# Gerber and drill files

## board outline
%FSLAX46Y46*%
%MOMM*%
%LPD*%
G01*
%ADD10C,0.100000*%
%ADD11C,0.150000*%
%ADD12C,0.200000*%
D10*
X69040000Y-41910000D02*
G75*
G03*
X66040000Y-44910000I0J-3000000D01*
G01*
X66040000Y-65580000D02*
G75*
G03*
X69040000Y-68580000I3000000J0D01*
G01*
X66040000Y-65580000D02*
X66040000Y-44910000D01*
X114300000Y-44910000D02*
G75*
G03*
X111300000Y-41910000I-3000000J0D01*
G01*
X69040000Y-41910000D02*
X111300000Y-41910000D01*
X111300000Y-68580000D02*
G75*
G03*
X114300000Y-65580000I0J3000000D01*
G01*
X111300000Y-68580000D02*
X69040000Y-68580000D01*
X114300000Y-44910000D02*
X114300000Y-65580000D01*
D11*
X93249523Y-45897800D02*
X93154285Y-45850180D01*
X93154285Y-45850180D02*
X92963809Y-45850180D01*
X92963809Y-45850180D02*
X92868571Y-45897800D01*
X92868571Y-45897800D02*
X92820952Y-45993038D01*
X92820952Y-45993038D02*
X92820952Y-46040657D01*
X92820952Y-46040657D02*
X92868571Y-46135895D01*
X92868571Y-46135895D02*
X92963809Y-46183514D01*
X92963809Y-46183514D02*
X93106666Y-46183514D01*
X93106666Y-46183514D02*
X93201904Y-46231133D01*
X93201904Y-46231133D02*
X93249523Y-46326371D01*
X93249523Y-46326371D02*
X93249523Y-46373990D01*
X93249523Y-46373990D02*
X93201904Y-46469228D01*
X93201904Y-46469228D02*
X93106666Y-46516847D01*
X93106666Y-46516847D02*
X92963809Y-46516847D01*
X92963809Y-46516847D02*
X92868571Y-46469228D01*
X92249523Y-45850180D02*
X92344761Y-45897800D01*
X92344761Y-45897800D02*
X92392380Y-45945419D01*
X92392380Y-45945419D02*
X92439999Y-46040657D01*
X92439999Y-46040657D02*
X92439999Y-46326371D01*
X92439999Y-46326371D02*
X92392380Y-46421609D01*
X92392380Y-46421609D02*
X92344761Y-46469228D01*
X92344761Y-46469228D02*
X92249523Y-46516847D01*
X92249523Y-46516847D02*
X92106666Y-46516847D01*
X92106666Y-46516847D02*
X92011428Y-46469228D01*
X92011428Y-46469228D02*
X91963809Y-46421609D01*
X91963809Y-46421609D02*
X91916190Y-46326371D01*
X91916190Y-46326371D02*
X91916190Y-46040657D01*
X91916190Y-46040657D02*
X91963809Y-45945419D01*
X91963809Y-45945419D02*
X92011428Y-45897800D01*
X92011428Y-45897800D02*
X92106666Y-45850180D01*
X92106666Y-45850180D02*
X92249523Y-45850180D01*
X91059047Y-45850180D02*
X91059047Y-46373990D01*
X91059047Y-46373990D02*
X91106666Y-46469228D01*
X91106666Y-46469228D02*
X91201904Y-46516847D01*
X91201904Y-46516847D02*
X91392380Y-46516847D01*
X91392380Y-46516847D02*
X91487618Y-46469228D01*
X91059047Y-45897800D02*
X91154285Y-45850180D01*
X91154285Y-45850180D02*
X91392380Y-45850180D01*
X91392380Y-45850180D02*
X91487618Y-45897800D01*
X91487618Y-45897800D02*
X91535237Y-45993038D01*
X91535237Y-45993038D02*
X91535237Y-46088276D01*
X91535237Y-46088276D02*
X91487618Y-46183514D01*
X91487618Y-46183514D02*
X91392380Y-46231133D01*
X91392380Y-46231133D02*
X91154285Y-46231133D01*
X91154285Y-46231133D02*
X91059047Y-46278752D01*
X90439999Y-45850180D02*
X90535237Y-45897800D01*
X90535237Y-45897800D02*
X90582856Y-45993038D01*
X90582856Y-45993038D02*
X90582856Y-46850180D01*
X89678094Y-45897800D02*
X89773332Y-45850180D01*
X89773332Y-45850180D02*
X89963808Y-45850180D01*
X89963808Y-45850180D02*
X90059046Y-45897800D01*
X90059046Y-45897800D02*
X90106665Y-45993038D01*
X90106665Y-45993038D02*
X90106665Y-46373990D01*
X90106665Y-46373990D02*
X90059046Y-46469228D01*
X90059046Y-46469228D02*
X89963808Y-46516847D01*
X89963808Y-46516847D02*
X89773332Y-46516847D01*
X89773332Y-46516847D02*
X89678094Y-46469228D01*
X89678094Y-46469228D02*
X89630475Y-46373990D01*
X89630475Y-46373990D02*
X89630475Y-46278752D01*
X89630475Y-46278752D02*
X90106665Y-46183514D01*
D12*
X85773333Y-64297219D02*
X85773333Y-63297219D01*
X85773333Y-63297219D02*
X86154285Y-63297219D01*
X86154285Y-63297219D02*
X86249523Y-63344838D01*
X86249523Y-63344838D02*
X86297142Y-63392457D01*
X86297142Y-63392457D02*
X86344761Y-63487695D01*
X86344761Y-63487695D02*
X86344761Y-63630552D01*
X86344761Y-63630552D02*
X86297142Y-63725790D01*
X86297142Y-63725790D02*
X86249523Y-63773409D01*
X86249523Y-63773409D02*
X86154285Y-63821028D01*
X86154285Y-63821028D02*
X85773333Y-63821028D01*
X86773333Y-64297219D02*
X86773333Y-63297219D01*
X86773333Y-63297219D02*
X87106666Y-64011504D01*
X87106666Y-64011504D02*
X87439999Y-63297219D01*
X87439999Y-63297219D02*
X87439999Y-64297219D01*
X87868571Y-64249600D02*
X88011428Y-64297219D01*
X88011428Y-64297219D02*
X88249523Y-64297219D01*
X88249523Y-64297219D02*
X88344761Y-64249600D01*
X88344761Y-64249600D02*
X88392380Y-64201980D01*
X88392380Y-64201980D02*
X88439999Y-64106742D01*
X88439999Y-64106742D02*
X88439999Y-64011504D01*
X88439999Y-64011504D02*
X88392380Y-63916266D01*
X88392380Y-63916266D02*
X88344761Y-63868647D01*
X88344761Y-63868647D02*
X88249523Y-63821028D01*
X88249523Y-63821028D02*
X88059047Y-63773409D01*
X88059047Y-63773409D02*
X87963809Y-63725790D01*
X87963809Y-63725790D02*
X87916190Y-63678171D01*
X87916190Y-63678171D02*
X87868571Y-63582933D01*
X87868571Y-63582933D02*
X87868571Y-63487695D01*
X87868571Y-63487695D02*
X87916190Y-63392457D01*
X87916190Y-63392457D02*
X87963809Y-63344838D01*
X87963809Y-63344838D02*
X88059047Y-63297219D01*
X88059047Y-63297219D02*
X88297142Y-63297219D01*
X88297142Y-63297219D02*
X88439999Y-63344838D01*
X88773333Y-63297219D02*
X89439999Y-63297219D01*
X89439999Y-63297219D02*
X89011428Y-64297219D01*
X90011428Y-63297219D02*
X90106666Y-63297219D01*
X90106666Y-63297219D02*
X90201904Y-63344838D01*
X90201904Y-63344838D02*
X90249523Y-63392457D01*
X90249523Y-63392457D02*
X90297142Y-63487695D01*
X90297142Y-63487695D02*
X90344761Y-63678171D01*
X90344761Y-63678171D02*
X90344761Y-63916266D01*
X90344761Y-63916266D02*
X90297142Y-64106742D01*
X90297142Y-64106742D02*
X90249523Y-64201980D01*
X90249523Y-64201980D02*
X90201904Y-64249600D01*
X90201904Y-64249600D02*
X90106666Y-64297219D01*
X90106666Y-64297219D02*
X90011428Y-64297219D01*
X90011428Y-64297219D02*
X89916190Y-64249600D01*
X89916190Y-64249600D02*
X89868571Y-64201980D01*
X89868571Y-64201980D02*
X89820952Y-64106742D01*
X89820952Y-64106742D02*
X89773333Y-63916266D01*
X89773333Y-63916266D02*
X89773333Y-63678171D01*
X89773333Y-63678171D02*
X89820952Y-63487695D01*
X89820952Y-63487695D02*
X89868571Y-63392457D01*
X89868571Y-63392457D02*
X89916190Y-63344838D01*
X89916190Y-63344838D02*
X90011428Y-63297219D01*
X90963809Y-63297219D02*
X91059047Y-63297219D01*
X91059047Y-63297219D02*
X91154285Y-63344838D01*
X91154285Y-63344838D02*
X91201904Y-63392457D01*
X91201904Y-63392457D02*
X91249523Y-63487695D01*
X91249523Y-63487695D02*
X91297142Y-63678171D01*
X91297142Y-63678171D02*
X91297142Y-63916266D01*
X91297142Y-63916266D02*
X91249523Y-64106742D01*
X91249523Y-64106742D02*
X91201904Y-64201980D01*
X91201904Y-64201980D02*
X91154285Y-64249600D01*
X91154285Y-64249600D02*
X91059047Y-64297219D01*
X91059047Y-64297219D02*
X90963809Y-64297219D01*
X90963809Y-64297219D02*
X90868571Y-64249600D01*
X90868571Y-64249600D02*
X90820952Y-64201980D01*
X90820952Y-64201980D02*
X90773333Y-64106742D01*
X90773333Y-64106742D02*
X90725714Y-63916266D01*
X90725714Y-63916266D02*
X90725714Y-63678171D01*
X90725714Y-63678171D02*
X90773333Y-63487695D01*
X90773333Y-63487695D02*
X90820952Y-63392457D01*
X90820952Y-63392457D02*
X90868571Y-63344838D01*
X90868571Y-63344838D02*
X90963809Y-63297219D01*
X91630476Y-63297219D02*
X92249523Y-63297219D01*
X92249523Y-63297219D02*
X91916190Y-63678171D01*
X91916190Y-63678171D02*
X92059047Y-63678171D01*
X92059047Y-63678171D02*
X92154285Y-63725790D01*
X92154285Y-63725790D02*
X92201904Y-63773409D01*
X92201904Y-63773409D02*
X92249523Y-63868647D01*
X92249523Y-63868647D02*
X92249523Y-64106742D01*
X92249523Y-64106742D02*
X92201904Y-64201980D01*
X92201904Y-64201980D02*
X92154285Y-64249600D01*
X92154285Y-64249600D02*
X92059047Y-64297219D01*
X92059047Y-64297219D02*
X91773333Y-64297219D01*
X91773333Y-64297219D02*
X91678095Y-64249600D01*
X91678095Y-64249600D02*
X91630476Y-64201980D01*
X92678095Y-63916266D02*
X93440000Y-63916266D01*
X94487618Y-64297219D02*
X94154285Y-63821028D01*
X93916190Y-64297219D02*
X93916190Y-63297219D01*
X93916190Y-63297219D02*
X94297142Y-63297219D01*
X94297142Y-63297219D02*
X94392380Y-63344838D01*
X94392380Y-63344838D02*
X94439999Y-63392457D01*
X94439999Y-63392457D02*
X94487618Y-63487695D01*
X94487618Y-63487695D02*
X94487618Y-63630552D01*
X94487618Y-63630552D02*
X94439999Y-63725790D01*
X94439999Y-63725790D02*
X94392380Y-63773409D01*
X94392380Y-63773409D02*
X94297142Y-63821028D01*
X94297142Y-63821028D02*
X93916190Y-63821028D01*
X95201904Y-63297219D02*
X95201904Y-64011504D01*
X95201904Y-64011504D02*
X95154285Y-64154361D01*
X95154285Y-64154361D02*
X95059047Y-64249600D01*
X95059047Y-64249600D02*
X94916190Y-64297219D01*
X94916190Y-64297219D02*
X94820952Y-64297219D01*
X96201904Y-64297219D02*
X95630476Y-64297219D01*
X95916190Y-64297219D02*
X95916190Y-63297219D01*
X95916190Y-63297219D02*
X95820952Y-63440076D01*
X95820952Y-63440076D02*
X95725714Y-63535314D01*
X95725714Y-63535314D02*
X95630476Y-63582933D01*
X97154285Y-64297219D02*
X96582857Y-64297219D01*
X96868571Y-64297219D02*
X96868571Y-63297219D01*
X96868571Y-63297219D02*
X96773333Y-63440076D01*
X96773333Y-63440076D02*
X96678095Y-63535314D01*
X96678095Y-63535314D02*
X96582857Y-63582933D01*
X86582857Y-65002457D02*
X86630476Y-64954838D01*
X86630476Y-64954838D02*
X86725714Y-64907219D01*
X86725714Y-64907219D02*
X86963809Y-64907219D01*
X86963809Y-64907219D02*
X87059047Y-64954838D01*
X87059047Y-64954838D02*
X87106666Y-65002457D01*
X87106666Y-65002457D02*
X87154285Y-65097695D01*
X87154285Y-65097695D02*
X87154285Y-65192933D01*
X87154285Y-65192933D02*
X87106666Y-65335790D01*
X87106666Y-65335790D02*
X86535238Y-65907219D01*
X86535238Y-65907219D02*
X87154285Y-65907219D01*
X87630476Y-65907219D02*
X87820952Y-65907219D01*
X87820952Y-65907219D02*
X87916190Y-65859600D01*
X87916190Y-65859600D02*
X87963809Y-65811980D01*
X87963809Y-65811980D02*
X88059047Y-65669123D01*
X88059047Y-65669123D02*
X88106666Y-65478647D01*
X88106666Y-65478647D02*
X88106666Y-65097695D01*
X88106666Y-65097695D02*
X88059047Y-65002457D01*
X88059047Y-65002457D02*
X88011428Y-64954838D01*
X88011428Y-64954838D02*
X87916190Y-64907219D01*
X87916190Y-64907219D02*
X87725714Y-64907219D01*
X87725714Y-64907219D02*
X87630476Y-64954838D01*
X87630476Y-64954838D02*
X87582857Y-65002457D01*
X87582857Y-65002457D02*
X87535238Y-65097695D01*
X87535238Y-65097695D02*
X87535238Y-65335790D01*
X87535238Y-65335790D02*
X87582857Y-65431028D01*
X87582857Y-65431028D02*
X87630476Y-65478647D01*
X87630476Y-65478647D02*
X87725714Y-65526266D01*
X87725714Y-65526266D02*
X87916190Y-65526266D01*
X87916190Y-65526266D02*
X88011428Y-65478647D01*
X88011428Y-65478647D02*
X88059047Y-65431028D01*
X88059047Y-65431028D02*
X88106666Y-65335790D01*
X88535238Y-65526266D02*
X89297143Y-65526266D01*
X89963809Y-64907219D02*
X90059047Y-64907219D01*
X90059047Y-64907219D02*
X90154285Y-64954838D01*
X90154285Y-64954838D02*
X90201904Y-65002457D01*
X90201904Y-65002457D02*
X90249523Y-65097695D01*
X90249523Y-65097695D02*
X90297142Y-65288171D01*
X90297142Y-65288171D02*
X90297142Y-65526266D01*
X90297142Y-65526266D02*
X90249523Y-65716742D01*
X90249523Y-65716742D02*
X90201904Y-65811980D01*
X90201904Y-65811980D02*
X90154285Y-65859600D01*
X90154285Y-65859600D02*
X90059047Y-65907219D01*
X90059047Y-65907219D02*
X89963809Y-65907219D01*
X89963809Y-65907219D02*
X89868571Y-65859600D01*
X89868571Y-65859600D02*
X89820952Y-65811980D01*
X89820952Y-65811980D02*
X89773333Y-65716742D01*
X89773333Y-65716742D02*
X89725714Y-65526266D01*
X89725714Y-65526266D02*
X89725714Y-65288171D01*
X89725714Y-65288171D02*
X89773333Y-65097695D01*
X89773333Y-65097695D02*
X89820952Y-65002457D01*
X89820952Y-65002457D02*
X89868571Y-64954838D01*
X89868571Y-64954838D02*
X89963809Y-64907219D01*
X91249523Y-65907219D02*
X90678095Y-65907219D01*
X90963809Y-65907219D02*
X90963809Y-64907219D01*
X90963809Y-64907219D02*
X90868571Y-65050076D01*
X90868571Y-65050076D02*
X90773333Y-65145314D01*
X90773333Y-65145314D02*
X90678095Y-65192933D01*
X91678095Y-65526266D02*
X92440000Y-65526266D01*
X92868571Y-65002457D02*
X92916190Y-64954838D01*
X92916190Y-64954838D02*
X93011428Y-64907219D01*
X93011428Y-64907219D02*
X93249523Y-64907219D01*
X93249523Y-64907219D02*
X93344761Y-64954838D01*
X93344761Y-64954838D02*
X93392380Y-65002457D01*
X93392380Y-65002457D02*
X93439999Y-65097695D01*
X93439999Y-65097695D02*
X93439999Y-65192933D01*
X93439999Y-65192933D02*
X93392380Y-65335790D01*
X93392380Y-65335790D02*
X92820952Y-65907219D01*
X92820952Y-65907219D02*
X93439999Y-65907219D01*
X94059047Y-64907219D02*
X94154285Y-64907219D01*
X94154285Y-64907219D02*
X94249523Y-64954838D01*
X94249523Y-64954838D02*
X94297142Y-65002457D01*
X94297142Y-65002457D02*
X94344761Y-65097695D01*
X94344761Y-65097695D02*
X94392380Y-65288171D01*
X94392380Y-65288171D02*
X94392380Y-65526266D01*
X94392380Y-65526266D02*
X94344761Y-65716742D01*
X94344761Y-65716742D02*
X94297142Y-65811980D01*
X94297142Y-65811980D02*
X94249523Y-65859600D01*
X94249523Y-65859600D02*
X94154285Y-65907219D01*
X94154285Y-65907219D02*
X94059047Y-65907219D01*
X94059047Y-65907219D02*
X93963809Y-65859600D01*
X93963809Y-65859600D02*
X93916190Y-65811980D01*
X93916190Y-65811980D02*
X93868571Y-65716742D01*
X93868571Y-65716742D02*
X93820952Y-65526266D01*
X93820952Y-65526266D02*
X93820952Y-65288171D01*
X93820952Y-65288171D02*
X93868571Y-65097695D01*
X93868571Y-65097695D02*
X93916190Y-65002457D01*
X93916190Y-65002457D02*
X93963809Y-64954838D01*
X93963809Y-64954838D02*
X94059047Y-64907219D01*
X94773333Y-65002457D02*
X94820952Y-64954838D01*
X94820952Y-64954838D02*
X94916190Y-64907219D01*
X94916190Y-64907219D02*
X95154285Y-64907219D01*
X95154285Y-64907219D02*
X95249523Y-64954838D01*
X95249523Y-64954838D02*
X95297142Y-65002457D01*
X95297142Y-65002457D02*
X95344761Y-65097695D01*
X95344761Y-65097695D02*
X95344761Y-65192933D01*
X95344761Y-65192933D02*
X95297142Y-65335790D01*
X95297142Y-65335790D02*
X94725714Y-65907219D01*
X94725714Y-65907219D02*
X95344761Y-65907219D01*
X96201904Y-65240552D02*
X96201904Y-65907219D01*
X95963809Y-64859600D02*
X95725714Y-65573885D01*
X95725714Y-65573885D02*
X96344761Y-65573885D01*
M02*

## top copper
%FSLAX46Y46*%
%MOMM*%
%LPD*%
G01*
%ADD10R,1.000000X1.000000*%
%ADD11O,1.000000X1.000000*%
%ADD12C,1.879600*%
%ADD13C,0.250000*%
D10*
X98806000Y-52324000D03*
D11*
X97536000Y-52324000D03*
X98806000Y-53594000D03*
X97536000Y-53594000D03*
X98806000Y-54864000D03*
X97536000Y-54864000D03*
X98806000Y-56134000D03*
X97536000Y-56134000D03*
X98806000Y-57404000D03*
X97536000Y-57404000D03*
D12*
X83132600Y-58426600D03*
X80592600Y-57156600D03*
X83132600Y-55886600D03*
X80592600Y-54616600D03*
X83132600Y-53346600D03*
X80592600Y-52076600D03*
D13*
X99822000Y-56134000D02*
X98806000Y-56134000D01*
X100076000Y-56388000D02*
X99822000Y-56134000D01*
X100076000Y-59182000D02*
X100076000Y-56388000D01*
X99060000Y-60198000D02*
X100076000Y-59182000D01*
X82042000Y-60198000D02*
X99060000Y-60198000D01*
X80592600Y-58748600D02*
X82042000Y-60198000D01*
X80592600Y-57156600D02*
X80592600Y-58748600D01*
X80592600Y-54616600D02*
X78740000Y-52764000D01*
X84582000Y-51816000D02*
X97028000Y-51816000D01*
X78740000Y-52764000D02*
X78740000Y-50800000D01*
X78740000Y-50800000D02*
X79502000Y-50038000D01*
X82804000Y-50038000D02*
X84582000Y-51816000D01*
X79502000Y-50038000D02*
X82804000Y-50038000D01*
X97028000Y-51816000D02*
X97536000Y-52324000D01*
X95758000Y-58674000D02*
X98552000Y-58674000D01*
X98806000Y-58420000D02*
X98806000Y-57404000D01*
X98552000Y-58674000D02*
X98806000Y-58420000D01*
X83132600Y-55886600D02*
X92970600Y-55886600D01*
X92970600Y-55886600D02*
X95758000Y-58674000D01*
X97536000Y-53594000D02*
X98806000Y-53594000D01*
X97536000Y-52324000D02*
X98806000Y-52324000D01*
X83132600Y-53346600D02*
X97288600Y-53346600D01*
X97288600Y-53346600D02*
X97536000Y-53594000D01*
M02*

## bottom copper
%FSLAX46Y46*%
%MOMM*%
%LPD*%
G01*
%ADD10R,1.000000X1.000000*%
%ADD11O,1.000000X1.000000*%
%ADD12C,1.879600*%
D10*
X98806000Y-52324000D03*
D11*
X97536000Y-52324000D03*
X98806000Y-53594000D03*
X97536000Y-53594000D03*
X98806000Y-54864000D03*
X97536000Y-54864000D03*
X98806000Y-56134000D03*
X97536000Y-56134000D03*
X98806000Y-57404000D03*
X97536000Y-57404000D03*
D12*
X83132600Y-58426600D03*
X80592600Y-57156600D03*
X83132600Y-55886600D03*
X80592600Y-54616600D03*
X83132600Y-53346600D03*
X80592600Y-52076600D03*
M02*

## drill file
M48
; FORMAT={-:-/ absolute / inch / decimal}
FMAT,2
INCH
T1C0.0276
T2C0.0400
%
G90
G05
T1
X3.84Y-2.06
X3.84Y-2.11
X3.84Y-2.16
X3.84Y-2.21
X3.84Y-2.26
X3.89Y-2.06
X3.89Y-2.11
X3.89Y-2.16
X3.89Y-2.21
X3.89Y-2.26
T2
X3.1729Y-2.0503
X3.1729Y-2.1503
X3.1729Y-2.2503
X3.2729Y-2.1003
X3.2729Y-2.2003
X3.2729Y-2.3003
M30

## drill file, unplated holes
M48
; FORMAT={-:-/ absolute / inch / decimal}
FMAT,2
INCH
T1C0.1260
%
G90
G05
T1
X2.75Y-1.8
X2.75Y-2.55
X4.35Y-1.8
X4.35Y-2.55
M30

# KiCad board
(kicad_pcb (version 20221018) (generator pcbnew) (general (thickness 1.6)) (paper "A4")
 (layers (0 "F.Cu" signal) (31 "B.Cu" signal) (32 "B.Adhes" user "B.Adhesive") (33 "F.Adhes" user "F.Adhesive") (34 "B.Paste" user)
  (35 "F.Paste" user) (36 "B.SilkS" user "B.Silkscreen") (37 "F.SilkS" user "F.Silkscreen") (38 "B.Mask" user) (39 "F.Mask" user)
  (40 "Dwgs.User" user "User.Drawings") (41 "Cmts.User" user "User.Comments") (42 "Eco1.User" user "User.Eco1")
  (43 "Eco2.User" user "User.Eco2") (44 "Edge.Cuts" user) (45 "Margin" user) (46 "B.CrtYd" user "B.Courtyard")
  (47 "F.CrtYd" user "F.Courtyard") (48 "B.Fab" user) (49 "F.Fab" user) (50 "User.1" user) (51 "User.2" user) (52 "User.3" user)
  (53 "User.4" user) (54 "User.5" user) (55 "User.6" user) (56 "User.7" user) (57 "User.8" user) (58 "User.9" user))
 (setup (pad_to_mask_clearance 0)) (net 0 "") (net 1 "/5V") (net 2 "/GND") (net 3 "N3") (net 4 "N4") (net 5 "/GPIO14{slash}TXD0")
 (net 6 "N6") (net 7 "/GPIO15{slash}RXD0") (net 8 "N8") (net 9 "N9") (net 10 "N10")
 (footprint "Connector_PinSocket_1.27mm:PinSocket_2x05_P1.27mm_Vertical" (layer "F.Cu") (at 98.806 52.324)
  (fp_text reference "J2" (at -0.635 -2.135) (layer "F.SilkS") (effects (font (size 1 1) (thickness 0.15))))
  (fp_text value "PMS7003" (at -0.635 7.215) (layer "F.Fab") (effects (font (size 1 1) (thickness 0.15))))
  (pad "1" thru_hole rect (at 0 0) (size 1 1) (drill 0.7) (layers "*.Cu" "*.Mask") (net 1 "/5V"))
  (pad "2" thru_hole oval (at -1.27 0) (size 1 1) (drill 0.7) (layers "*.Cu" "*.Mask") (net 1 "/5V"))
  (pad "3" thru_hole oval (at 0 1.27) (size 1 1) (drill 0.7) (layers "*.Cu" "*.Mask") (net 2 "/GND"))
  (pad "4" thru_hole oval (at -1.27 1.27) (size 1 1) (drill 0.7) (layers "*.Cu" "*.Mask") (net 2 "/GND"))
  (pad "5" thru_hole oval (at 0 2.54) (size 1 1) (drill 0.7) (layers "*.Cu" "*.Mask") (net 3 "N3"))
  (pad "6" thru_hole oval (at -1.27 2.54) (size 1 1) (drill 0.7) (layers "*.Cu" "*.Mask") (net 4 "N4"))
  (pad "7" thru_hole oval (at 0 3.81) (size 1 1) (drill 0.7) (layers "*.Cu" "*.Mask") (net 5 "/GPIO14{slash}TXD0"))
  (pad "8" thru_hole oval (at -1.27 3.81) (size 1 1) (drill 0.7) (layers "*.Cu" "*.Mask") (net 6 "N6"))
  (pad "9" thru_hole oval (at 0 5.08) (size 1 1) (drill 0.7) (layers "*.Cu" "*.Mask") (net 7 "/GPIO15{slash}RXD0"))
  (pad "10" thru_hole oval (at -1.27 5.08) (size 1 1) (drill 0.7) (layers "*.Cu" "*.Mask") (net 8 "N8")))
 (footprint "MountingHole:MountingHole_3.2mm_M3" (layer "F.Cu") (at 110.49 45.72)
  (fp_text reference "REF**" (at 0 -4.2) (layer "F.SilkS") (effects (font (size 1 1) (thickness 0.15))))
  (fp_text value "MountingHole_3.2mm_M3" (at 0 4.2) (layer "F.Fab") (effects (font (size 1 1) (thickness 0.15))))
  (pad "" np_thru_hole circle (at 0 0) (size 3.2 3.2) (drill 3.2) (layers "*.Cu" "*.Mask")))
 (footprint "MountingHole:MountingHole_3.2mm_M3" (layer "F.Cu") (at 69.85 45.72)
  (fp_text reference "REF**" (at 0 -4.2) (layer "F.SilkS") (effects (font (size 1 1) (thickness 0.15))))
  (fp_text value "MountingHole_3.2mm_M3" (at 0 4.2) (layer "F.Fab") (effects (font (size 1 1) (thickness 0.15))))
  (pad "" np_thru_hole circle (at 0 0) (size 3.2 3.2) (drill 3.2) (layers "*.Cu" "*.Mask")))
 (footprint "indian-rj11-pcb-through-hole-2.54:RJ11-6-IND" (layer "F.Cu") (at 78.7326 55.2566 -90)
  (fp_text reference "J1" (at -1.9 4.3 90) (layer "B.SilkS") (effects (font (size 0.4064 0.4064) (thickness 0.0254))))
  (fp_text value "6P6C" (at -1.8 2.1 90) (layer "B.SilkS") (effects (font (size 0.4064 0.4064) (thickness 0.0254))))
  (pad "1" thru_hole circle (at 3.17 -4.4 90) (size 1.8796 1.8796) (drill 1.016) (layers "F&B.Cu" "F.Paste" "F.SilkS" "F.Mask") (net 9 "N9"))
  (pad "2" thru_hole circle (at 1.9 -1.86 90) (size 1.8796 1.8796) (drill 1.016) (layers "F&B.Cu" "F.Paste" "F.SilkS" "F.Mask")
   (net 5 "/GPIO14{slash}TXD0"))
  (pad "3" thru_hole circle (at 0.63 -4.4 90) (size 1.8796 1.8796) (drill 1.016) (layers "F&B.Cu" "F.Paste" "F.SilkS" "F.Mask")
   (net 7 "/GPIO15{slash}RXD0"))
  (pad "4" thru_hole circle (at -0.64 -1.86 90) (size 1.8796 1.8796) (drill 1.016) (layers "F&B.Cu" "F.Paste" "F.SilkS" "F.Mask")
   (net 1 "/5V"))
  (pad "5" thru_hole circle (at -1.91 -4.4 90) (size 1.8796 1.8796) (drill 1.016) (layers "F&B.Cu" "F.Paste" "F.SilkS" "F.Mask")
   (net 2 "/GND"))
  (pad "6" thru_hole circle (at -3.18 -1.86 90) (size 1.8796 1.8796) (drill 1.016) (layers "F&B.Cu" "F.Paste" "F.SilkS" "F.Mask")
   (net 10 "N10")))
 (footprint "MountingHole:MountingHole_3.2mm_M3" (layer "F.Cu") (at 69.85 64.77)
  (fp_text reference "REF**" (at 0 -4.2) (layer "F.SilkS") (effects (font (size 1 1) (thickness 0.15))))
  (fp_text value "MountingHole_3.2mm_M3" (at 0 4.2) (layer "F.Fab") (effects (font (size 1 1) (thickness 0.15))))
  (pad "" np_thru_hole circle (at 0 0) (size 3.2 3.2) (drill 3.2) (layers "*.Cu" "*.Mask")))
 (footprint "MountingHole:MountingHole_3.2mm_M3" (layer "F.Cu") (at 110.49 64.77)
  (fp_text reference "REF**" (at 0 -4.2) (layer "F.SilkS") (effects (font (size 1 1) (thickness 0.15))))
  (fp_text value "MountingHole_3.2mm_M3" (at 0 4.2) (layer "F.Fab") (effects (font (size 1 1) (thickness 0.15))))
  (pad "" np_thru_hole circle (at 0 0) (size 3.2 3.2) (drill 3.2) (layers "*.Cu" "*.Mask")))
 (gr_line (start 69.04 41.91) (end 111.3 41.91) (stroke (width 0.1) (type default)) (layer "Edge.Cuts"))
 (gr_arc (start 69.04 68.58) (mid 66.91868 67.70132) (end 66.04 65.58) (stroke (width 0.1) (type default)) (layer "Edge.Cuts"))
 (gr_arc (start 114.3 65.58) (mid 113.42132 67.70132) (end 111.3 68.58) (stroke (width 0.1) (type default)) (layer "Edge.Cuts"))
 (gr_line (start 111.3 68.58) (end 69.04 68.58) (stroke (width 0.1) (type default)) (layer "Edge.Cuts"))
 (gr_arc (start 66.04 44.91) (mid 66.91868 42.78868) (end 69.04 41.91) (stroke (width 0.1) (type default)) (layer "Edge.Cuts"))
 (gr_arc (start 111.3 41.91) (mid 113.42132 42.78868) (end 114.3 44.91) (stroke (width 0.1) (type default)) (layer "Edge.Cuts"))
 (gr_line (start 66.04 65.58) (end 66.04 44.91) (stroke (width 0.1) (type default)) (layer "Edge.Cuts"))
 (gr_line (start 114.3 44.91) (end 114.3 65.58) (stroke (width 0.1) (type default)) (layer "Edge.Cuts"))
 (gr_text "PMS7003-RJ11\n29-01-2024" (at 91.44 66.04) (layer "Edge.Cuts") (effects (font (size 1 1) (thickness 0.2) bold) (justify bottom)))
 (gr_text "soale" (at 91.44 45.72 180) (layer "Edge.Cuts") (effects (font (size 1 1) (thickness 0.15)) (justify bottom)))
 (segment (start 82.042 60.198) (end 99.06 60.198) (width 0.25) (layer "F.Cu") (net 5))
 (segment (start 99.822 56.134) (end 98.806 56.134) (width 0.25) (layer "F.Cu") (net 5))
 (segment (start 100.076 56.388) (end 99.822 56.134) (width 0.25) (layer "F.Cu") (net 5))
 (segment (start 99.06 60.198) (end 100.076 59.182) (width 0.25) (layer "F.Cu") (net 5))
 (segment (start 80.5926 57.1566) (end 80.5926 58.7486) (width 0.25) (layer "F.Cu") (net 5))
 (segment (start 100.076 59.182) (end 100.076 56.388) (width 0.25) (layer "F.Cu") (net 5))
 (segment (start 80.5926 58.7486) (end 82.042 60.198) (width 0.25) (layer "F.Cu") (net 5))
 (segment (start 83.1326 55.8866) (end 92.9706 55.8866) (width 0.25) (layer "F.Cu") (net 7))
 (segment (start 95.758 58.674) (end 98.552 58.674) (width 0.25) (layer "F.Cu") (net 7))
 (segment (start 98.552 58.674) (end 98.806 58.42) (width 0.25) (layer "F.Cu") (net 7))
 (segment (start 92.9706 55.8866) (end 95.758 58.674) (width 0.25) (layer "F.Cu") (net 7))
 (segment (start 98.806 58.42) (end 98.806 57.404) (width 0.25) (layer "F.Cu") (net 7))
 (segment (start 78.74 52.764) (end 78.74 50.8) (width 0.25) (layer "F.Cu") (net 1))
 (segment (start 78.74 50.8) (end 79.502 50.038) (width 0.25) (layer "F.Cu") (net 1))
 (segment (start 79.502 50.038) (end 82.804 50.038) (width 0.25) (layer "F.Cu") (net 1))
 (segment (start 82.804 50.038) (end 84.582 51.816) (width 0.25) (layer "F.Cu") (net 1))
 (segment (start 97.536 52.324) (end 98.806 52.324) (width 0.25) (layer "F.Cu") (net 1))
 (segment (start 97.028 51.816) (end 97.536 52.324) (width 0.25) (layer "F.Cu") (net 1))
 (segment (start 80.5926 54.6166) (end 78.74 52.764) (width 0.25) (layer "F.Cu") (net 1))
 (segment (start 84.582 51.816) (end 97.028 51.816) (width 0.25) (layer "F.Cu") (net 1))
 (segment (start 83.1326 53.3466) (end 97.2886 53.3466) (width 0.25) (layer "F.Cu") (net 2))
 (segment (start 97.2886 53.3466) (end 97.536 53.594) (width 0.25) (layer "F.Cu") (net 2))
 (segment (start 97.536 53.594) (end 98.806 53.594) (width 0.25) (layer "F.Cu") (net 2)))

